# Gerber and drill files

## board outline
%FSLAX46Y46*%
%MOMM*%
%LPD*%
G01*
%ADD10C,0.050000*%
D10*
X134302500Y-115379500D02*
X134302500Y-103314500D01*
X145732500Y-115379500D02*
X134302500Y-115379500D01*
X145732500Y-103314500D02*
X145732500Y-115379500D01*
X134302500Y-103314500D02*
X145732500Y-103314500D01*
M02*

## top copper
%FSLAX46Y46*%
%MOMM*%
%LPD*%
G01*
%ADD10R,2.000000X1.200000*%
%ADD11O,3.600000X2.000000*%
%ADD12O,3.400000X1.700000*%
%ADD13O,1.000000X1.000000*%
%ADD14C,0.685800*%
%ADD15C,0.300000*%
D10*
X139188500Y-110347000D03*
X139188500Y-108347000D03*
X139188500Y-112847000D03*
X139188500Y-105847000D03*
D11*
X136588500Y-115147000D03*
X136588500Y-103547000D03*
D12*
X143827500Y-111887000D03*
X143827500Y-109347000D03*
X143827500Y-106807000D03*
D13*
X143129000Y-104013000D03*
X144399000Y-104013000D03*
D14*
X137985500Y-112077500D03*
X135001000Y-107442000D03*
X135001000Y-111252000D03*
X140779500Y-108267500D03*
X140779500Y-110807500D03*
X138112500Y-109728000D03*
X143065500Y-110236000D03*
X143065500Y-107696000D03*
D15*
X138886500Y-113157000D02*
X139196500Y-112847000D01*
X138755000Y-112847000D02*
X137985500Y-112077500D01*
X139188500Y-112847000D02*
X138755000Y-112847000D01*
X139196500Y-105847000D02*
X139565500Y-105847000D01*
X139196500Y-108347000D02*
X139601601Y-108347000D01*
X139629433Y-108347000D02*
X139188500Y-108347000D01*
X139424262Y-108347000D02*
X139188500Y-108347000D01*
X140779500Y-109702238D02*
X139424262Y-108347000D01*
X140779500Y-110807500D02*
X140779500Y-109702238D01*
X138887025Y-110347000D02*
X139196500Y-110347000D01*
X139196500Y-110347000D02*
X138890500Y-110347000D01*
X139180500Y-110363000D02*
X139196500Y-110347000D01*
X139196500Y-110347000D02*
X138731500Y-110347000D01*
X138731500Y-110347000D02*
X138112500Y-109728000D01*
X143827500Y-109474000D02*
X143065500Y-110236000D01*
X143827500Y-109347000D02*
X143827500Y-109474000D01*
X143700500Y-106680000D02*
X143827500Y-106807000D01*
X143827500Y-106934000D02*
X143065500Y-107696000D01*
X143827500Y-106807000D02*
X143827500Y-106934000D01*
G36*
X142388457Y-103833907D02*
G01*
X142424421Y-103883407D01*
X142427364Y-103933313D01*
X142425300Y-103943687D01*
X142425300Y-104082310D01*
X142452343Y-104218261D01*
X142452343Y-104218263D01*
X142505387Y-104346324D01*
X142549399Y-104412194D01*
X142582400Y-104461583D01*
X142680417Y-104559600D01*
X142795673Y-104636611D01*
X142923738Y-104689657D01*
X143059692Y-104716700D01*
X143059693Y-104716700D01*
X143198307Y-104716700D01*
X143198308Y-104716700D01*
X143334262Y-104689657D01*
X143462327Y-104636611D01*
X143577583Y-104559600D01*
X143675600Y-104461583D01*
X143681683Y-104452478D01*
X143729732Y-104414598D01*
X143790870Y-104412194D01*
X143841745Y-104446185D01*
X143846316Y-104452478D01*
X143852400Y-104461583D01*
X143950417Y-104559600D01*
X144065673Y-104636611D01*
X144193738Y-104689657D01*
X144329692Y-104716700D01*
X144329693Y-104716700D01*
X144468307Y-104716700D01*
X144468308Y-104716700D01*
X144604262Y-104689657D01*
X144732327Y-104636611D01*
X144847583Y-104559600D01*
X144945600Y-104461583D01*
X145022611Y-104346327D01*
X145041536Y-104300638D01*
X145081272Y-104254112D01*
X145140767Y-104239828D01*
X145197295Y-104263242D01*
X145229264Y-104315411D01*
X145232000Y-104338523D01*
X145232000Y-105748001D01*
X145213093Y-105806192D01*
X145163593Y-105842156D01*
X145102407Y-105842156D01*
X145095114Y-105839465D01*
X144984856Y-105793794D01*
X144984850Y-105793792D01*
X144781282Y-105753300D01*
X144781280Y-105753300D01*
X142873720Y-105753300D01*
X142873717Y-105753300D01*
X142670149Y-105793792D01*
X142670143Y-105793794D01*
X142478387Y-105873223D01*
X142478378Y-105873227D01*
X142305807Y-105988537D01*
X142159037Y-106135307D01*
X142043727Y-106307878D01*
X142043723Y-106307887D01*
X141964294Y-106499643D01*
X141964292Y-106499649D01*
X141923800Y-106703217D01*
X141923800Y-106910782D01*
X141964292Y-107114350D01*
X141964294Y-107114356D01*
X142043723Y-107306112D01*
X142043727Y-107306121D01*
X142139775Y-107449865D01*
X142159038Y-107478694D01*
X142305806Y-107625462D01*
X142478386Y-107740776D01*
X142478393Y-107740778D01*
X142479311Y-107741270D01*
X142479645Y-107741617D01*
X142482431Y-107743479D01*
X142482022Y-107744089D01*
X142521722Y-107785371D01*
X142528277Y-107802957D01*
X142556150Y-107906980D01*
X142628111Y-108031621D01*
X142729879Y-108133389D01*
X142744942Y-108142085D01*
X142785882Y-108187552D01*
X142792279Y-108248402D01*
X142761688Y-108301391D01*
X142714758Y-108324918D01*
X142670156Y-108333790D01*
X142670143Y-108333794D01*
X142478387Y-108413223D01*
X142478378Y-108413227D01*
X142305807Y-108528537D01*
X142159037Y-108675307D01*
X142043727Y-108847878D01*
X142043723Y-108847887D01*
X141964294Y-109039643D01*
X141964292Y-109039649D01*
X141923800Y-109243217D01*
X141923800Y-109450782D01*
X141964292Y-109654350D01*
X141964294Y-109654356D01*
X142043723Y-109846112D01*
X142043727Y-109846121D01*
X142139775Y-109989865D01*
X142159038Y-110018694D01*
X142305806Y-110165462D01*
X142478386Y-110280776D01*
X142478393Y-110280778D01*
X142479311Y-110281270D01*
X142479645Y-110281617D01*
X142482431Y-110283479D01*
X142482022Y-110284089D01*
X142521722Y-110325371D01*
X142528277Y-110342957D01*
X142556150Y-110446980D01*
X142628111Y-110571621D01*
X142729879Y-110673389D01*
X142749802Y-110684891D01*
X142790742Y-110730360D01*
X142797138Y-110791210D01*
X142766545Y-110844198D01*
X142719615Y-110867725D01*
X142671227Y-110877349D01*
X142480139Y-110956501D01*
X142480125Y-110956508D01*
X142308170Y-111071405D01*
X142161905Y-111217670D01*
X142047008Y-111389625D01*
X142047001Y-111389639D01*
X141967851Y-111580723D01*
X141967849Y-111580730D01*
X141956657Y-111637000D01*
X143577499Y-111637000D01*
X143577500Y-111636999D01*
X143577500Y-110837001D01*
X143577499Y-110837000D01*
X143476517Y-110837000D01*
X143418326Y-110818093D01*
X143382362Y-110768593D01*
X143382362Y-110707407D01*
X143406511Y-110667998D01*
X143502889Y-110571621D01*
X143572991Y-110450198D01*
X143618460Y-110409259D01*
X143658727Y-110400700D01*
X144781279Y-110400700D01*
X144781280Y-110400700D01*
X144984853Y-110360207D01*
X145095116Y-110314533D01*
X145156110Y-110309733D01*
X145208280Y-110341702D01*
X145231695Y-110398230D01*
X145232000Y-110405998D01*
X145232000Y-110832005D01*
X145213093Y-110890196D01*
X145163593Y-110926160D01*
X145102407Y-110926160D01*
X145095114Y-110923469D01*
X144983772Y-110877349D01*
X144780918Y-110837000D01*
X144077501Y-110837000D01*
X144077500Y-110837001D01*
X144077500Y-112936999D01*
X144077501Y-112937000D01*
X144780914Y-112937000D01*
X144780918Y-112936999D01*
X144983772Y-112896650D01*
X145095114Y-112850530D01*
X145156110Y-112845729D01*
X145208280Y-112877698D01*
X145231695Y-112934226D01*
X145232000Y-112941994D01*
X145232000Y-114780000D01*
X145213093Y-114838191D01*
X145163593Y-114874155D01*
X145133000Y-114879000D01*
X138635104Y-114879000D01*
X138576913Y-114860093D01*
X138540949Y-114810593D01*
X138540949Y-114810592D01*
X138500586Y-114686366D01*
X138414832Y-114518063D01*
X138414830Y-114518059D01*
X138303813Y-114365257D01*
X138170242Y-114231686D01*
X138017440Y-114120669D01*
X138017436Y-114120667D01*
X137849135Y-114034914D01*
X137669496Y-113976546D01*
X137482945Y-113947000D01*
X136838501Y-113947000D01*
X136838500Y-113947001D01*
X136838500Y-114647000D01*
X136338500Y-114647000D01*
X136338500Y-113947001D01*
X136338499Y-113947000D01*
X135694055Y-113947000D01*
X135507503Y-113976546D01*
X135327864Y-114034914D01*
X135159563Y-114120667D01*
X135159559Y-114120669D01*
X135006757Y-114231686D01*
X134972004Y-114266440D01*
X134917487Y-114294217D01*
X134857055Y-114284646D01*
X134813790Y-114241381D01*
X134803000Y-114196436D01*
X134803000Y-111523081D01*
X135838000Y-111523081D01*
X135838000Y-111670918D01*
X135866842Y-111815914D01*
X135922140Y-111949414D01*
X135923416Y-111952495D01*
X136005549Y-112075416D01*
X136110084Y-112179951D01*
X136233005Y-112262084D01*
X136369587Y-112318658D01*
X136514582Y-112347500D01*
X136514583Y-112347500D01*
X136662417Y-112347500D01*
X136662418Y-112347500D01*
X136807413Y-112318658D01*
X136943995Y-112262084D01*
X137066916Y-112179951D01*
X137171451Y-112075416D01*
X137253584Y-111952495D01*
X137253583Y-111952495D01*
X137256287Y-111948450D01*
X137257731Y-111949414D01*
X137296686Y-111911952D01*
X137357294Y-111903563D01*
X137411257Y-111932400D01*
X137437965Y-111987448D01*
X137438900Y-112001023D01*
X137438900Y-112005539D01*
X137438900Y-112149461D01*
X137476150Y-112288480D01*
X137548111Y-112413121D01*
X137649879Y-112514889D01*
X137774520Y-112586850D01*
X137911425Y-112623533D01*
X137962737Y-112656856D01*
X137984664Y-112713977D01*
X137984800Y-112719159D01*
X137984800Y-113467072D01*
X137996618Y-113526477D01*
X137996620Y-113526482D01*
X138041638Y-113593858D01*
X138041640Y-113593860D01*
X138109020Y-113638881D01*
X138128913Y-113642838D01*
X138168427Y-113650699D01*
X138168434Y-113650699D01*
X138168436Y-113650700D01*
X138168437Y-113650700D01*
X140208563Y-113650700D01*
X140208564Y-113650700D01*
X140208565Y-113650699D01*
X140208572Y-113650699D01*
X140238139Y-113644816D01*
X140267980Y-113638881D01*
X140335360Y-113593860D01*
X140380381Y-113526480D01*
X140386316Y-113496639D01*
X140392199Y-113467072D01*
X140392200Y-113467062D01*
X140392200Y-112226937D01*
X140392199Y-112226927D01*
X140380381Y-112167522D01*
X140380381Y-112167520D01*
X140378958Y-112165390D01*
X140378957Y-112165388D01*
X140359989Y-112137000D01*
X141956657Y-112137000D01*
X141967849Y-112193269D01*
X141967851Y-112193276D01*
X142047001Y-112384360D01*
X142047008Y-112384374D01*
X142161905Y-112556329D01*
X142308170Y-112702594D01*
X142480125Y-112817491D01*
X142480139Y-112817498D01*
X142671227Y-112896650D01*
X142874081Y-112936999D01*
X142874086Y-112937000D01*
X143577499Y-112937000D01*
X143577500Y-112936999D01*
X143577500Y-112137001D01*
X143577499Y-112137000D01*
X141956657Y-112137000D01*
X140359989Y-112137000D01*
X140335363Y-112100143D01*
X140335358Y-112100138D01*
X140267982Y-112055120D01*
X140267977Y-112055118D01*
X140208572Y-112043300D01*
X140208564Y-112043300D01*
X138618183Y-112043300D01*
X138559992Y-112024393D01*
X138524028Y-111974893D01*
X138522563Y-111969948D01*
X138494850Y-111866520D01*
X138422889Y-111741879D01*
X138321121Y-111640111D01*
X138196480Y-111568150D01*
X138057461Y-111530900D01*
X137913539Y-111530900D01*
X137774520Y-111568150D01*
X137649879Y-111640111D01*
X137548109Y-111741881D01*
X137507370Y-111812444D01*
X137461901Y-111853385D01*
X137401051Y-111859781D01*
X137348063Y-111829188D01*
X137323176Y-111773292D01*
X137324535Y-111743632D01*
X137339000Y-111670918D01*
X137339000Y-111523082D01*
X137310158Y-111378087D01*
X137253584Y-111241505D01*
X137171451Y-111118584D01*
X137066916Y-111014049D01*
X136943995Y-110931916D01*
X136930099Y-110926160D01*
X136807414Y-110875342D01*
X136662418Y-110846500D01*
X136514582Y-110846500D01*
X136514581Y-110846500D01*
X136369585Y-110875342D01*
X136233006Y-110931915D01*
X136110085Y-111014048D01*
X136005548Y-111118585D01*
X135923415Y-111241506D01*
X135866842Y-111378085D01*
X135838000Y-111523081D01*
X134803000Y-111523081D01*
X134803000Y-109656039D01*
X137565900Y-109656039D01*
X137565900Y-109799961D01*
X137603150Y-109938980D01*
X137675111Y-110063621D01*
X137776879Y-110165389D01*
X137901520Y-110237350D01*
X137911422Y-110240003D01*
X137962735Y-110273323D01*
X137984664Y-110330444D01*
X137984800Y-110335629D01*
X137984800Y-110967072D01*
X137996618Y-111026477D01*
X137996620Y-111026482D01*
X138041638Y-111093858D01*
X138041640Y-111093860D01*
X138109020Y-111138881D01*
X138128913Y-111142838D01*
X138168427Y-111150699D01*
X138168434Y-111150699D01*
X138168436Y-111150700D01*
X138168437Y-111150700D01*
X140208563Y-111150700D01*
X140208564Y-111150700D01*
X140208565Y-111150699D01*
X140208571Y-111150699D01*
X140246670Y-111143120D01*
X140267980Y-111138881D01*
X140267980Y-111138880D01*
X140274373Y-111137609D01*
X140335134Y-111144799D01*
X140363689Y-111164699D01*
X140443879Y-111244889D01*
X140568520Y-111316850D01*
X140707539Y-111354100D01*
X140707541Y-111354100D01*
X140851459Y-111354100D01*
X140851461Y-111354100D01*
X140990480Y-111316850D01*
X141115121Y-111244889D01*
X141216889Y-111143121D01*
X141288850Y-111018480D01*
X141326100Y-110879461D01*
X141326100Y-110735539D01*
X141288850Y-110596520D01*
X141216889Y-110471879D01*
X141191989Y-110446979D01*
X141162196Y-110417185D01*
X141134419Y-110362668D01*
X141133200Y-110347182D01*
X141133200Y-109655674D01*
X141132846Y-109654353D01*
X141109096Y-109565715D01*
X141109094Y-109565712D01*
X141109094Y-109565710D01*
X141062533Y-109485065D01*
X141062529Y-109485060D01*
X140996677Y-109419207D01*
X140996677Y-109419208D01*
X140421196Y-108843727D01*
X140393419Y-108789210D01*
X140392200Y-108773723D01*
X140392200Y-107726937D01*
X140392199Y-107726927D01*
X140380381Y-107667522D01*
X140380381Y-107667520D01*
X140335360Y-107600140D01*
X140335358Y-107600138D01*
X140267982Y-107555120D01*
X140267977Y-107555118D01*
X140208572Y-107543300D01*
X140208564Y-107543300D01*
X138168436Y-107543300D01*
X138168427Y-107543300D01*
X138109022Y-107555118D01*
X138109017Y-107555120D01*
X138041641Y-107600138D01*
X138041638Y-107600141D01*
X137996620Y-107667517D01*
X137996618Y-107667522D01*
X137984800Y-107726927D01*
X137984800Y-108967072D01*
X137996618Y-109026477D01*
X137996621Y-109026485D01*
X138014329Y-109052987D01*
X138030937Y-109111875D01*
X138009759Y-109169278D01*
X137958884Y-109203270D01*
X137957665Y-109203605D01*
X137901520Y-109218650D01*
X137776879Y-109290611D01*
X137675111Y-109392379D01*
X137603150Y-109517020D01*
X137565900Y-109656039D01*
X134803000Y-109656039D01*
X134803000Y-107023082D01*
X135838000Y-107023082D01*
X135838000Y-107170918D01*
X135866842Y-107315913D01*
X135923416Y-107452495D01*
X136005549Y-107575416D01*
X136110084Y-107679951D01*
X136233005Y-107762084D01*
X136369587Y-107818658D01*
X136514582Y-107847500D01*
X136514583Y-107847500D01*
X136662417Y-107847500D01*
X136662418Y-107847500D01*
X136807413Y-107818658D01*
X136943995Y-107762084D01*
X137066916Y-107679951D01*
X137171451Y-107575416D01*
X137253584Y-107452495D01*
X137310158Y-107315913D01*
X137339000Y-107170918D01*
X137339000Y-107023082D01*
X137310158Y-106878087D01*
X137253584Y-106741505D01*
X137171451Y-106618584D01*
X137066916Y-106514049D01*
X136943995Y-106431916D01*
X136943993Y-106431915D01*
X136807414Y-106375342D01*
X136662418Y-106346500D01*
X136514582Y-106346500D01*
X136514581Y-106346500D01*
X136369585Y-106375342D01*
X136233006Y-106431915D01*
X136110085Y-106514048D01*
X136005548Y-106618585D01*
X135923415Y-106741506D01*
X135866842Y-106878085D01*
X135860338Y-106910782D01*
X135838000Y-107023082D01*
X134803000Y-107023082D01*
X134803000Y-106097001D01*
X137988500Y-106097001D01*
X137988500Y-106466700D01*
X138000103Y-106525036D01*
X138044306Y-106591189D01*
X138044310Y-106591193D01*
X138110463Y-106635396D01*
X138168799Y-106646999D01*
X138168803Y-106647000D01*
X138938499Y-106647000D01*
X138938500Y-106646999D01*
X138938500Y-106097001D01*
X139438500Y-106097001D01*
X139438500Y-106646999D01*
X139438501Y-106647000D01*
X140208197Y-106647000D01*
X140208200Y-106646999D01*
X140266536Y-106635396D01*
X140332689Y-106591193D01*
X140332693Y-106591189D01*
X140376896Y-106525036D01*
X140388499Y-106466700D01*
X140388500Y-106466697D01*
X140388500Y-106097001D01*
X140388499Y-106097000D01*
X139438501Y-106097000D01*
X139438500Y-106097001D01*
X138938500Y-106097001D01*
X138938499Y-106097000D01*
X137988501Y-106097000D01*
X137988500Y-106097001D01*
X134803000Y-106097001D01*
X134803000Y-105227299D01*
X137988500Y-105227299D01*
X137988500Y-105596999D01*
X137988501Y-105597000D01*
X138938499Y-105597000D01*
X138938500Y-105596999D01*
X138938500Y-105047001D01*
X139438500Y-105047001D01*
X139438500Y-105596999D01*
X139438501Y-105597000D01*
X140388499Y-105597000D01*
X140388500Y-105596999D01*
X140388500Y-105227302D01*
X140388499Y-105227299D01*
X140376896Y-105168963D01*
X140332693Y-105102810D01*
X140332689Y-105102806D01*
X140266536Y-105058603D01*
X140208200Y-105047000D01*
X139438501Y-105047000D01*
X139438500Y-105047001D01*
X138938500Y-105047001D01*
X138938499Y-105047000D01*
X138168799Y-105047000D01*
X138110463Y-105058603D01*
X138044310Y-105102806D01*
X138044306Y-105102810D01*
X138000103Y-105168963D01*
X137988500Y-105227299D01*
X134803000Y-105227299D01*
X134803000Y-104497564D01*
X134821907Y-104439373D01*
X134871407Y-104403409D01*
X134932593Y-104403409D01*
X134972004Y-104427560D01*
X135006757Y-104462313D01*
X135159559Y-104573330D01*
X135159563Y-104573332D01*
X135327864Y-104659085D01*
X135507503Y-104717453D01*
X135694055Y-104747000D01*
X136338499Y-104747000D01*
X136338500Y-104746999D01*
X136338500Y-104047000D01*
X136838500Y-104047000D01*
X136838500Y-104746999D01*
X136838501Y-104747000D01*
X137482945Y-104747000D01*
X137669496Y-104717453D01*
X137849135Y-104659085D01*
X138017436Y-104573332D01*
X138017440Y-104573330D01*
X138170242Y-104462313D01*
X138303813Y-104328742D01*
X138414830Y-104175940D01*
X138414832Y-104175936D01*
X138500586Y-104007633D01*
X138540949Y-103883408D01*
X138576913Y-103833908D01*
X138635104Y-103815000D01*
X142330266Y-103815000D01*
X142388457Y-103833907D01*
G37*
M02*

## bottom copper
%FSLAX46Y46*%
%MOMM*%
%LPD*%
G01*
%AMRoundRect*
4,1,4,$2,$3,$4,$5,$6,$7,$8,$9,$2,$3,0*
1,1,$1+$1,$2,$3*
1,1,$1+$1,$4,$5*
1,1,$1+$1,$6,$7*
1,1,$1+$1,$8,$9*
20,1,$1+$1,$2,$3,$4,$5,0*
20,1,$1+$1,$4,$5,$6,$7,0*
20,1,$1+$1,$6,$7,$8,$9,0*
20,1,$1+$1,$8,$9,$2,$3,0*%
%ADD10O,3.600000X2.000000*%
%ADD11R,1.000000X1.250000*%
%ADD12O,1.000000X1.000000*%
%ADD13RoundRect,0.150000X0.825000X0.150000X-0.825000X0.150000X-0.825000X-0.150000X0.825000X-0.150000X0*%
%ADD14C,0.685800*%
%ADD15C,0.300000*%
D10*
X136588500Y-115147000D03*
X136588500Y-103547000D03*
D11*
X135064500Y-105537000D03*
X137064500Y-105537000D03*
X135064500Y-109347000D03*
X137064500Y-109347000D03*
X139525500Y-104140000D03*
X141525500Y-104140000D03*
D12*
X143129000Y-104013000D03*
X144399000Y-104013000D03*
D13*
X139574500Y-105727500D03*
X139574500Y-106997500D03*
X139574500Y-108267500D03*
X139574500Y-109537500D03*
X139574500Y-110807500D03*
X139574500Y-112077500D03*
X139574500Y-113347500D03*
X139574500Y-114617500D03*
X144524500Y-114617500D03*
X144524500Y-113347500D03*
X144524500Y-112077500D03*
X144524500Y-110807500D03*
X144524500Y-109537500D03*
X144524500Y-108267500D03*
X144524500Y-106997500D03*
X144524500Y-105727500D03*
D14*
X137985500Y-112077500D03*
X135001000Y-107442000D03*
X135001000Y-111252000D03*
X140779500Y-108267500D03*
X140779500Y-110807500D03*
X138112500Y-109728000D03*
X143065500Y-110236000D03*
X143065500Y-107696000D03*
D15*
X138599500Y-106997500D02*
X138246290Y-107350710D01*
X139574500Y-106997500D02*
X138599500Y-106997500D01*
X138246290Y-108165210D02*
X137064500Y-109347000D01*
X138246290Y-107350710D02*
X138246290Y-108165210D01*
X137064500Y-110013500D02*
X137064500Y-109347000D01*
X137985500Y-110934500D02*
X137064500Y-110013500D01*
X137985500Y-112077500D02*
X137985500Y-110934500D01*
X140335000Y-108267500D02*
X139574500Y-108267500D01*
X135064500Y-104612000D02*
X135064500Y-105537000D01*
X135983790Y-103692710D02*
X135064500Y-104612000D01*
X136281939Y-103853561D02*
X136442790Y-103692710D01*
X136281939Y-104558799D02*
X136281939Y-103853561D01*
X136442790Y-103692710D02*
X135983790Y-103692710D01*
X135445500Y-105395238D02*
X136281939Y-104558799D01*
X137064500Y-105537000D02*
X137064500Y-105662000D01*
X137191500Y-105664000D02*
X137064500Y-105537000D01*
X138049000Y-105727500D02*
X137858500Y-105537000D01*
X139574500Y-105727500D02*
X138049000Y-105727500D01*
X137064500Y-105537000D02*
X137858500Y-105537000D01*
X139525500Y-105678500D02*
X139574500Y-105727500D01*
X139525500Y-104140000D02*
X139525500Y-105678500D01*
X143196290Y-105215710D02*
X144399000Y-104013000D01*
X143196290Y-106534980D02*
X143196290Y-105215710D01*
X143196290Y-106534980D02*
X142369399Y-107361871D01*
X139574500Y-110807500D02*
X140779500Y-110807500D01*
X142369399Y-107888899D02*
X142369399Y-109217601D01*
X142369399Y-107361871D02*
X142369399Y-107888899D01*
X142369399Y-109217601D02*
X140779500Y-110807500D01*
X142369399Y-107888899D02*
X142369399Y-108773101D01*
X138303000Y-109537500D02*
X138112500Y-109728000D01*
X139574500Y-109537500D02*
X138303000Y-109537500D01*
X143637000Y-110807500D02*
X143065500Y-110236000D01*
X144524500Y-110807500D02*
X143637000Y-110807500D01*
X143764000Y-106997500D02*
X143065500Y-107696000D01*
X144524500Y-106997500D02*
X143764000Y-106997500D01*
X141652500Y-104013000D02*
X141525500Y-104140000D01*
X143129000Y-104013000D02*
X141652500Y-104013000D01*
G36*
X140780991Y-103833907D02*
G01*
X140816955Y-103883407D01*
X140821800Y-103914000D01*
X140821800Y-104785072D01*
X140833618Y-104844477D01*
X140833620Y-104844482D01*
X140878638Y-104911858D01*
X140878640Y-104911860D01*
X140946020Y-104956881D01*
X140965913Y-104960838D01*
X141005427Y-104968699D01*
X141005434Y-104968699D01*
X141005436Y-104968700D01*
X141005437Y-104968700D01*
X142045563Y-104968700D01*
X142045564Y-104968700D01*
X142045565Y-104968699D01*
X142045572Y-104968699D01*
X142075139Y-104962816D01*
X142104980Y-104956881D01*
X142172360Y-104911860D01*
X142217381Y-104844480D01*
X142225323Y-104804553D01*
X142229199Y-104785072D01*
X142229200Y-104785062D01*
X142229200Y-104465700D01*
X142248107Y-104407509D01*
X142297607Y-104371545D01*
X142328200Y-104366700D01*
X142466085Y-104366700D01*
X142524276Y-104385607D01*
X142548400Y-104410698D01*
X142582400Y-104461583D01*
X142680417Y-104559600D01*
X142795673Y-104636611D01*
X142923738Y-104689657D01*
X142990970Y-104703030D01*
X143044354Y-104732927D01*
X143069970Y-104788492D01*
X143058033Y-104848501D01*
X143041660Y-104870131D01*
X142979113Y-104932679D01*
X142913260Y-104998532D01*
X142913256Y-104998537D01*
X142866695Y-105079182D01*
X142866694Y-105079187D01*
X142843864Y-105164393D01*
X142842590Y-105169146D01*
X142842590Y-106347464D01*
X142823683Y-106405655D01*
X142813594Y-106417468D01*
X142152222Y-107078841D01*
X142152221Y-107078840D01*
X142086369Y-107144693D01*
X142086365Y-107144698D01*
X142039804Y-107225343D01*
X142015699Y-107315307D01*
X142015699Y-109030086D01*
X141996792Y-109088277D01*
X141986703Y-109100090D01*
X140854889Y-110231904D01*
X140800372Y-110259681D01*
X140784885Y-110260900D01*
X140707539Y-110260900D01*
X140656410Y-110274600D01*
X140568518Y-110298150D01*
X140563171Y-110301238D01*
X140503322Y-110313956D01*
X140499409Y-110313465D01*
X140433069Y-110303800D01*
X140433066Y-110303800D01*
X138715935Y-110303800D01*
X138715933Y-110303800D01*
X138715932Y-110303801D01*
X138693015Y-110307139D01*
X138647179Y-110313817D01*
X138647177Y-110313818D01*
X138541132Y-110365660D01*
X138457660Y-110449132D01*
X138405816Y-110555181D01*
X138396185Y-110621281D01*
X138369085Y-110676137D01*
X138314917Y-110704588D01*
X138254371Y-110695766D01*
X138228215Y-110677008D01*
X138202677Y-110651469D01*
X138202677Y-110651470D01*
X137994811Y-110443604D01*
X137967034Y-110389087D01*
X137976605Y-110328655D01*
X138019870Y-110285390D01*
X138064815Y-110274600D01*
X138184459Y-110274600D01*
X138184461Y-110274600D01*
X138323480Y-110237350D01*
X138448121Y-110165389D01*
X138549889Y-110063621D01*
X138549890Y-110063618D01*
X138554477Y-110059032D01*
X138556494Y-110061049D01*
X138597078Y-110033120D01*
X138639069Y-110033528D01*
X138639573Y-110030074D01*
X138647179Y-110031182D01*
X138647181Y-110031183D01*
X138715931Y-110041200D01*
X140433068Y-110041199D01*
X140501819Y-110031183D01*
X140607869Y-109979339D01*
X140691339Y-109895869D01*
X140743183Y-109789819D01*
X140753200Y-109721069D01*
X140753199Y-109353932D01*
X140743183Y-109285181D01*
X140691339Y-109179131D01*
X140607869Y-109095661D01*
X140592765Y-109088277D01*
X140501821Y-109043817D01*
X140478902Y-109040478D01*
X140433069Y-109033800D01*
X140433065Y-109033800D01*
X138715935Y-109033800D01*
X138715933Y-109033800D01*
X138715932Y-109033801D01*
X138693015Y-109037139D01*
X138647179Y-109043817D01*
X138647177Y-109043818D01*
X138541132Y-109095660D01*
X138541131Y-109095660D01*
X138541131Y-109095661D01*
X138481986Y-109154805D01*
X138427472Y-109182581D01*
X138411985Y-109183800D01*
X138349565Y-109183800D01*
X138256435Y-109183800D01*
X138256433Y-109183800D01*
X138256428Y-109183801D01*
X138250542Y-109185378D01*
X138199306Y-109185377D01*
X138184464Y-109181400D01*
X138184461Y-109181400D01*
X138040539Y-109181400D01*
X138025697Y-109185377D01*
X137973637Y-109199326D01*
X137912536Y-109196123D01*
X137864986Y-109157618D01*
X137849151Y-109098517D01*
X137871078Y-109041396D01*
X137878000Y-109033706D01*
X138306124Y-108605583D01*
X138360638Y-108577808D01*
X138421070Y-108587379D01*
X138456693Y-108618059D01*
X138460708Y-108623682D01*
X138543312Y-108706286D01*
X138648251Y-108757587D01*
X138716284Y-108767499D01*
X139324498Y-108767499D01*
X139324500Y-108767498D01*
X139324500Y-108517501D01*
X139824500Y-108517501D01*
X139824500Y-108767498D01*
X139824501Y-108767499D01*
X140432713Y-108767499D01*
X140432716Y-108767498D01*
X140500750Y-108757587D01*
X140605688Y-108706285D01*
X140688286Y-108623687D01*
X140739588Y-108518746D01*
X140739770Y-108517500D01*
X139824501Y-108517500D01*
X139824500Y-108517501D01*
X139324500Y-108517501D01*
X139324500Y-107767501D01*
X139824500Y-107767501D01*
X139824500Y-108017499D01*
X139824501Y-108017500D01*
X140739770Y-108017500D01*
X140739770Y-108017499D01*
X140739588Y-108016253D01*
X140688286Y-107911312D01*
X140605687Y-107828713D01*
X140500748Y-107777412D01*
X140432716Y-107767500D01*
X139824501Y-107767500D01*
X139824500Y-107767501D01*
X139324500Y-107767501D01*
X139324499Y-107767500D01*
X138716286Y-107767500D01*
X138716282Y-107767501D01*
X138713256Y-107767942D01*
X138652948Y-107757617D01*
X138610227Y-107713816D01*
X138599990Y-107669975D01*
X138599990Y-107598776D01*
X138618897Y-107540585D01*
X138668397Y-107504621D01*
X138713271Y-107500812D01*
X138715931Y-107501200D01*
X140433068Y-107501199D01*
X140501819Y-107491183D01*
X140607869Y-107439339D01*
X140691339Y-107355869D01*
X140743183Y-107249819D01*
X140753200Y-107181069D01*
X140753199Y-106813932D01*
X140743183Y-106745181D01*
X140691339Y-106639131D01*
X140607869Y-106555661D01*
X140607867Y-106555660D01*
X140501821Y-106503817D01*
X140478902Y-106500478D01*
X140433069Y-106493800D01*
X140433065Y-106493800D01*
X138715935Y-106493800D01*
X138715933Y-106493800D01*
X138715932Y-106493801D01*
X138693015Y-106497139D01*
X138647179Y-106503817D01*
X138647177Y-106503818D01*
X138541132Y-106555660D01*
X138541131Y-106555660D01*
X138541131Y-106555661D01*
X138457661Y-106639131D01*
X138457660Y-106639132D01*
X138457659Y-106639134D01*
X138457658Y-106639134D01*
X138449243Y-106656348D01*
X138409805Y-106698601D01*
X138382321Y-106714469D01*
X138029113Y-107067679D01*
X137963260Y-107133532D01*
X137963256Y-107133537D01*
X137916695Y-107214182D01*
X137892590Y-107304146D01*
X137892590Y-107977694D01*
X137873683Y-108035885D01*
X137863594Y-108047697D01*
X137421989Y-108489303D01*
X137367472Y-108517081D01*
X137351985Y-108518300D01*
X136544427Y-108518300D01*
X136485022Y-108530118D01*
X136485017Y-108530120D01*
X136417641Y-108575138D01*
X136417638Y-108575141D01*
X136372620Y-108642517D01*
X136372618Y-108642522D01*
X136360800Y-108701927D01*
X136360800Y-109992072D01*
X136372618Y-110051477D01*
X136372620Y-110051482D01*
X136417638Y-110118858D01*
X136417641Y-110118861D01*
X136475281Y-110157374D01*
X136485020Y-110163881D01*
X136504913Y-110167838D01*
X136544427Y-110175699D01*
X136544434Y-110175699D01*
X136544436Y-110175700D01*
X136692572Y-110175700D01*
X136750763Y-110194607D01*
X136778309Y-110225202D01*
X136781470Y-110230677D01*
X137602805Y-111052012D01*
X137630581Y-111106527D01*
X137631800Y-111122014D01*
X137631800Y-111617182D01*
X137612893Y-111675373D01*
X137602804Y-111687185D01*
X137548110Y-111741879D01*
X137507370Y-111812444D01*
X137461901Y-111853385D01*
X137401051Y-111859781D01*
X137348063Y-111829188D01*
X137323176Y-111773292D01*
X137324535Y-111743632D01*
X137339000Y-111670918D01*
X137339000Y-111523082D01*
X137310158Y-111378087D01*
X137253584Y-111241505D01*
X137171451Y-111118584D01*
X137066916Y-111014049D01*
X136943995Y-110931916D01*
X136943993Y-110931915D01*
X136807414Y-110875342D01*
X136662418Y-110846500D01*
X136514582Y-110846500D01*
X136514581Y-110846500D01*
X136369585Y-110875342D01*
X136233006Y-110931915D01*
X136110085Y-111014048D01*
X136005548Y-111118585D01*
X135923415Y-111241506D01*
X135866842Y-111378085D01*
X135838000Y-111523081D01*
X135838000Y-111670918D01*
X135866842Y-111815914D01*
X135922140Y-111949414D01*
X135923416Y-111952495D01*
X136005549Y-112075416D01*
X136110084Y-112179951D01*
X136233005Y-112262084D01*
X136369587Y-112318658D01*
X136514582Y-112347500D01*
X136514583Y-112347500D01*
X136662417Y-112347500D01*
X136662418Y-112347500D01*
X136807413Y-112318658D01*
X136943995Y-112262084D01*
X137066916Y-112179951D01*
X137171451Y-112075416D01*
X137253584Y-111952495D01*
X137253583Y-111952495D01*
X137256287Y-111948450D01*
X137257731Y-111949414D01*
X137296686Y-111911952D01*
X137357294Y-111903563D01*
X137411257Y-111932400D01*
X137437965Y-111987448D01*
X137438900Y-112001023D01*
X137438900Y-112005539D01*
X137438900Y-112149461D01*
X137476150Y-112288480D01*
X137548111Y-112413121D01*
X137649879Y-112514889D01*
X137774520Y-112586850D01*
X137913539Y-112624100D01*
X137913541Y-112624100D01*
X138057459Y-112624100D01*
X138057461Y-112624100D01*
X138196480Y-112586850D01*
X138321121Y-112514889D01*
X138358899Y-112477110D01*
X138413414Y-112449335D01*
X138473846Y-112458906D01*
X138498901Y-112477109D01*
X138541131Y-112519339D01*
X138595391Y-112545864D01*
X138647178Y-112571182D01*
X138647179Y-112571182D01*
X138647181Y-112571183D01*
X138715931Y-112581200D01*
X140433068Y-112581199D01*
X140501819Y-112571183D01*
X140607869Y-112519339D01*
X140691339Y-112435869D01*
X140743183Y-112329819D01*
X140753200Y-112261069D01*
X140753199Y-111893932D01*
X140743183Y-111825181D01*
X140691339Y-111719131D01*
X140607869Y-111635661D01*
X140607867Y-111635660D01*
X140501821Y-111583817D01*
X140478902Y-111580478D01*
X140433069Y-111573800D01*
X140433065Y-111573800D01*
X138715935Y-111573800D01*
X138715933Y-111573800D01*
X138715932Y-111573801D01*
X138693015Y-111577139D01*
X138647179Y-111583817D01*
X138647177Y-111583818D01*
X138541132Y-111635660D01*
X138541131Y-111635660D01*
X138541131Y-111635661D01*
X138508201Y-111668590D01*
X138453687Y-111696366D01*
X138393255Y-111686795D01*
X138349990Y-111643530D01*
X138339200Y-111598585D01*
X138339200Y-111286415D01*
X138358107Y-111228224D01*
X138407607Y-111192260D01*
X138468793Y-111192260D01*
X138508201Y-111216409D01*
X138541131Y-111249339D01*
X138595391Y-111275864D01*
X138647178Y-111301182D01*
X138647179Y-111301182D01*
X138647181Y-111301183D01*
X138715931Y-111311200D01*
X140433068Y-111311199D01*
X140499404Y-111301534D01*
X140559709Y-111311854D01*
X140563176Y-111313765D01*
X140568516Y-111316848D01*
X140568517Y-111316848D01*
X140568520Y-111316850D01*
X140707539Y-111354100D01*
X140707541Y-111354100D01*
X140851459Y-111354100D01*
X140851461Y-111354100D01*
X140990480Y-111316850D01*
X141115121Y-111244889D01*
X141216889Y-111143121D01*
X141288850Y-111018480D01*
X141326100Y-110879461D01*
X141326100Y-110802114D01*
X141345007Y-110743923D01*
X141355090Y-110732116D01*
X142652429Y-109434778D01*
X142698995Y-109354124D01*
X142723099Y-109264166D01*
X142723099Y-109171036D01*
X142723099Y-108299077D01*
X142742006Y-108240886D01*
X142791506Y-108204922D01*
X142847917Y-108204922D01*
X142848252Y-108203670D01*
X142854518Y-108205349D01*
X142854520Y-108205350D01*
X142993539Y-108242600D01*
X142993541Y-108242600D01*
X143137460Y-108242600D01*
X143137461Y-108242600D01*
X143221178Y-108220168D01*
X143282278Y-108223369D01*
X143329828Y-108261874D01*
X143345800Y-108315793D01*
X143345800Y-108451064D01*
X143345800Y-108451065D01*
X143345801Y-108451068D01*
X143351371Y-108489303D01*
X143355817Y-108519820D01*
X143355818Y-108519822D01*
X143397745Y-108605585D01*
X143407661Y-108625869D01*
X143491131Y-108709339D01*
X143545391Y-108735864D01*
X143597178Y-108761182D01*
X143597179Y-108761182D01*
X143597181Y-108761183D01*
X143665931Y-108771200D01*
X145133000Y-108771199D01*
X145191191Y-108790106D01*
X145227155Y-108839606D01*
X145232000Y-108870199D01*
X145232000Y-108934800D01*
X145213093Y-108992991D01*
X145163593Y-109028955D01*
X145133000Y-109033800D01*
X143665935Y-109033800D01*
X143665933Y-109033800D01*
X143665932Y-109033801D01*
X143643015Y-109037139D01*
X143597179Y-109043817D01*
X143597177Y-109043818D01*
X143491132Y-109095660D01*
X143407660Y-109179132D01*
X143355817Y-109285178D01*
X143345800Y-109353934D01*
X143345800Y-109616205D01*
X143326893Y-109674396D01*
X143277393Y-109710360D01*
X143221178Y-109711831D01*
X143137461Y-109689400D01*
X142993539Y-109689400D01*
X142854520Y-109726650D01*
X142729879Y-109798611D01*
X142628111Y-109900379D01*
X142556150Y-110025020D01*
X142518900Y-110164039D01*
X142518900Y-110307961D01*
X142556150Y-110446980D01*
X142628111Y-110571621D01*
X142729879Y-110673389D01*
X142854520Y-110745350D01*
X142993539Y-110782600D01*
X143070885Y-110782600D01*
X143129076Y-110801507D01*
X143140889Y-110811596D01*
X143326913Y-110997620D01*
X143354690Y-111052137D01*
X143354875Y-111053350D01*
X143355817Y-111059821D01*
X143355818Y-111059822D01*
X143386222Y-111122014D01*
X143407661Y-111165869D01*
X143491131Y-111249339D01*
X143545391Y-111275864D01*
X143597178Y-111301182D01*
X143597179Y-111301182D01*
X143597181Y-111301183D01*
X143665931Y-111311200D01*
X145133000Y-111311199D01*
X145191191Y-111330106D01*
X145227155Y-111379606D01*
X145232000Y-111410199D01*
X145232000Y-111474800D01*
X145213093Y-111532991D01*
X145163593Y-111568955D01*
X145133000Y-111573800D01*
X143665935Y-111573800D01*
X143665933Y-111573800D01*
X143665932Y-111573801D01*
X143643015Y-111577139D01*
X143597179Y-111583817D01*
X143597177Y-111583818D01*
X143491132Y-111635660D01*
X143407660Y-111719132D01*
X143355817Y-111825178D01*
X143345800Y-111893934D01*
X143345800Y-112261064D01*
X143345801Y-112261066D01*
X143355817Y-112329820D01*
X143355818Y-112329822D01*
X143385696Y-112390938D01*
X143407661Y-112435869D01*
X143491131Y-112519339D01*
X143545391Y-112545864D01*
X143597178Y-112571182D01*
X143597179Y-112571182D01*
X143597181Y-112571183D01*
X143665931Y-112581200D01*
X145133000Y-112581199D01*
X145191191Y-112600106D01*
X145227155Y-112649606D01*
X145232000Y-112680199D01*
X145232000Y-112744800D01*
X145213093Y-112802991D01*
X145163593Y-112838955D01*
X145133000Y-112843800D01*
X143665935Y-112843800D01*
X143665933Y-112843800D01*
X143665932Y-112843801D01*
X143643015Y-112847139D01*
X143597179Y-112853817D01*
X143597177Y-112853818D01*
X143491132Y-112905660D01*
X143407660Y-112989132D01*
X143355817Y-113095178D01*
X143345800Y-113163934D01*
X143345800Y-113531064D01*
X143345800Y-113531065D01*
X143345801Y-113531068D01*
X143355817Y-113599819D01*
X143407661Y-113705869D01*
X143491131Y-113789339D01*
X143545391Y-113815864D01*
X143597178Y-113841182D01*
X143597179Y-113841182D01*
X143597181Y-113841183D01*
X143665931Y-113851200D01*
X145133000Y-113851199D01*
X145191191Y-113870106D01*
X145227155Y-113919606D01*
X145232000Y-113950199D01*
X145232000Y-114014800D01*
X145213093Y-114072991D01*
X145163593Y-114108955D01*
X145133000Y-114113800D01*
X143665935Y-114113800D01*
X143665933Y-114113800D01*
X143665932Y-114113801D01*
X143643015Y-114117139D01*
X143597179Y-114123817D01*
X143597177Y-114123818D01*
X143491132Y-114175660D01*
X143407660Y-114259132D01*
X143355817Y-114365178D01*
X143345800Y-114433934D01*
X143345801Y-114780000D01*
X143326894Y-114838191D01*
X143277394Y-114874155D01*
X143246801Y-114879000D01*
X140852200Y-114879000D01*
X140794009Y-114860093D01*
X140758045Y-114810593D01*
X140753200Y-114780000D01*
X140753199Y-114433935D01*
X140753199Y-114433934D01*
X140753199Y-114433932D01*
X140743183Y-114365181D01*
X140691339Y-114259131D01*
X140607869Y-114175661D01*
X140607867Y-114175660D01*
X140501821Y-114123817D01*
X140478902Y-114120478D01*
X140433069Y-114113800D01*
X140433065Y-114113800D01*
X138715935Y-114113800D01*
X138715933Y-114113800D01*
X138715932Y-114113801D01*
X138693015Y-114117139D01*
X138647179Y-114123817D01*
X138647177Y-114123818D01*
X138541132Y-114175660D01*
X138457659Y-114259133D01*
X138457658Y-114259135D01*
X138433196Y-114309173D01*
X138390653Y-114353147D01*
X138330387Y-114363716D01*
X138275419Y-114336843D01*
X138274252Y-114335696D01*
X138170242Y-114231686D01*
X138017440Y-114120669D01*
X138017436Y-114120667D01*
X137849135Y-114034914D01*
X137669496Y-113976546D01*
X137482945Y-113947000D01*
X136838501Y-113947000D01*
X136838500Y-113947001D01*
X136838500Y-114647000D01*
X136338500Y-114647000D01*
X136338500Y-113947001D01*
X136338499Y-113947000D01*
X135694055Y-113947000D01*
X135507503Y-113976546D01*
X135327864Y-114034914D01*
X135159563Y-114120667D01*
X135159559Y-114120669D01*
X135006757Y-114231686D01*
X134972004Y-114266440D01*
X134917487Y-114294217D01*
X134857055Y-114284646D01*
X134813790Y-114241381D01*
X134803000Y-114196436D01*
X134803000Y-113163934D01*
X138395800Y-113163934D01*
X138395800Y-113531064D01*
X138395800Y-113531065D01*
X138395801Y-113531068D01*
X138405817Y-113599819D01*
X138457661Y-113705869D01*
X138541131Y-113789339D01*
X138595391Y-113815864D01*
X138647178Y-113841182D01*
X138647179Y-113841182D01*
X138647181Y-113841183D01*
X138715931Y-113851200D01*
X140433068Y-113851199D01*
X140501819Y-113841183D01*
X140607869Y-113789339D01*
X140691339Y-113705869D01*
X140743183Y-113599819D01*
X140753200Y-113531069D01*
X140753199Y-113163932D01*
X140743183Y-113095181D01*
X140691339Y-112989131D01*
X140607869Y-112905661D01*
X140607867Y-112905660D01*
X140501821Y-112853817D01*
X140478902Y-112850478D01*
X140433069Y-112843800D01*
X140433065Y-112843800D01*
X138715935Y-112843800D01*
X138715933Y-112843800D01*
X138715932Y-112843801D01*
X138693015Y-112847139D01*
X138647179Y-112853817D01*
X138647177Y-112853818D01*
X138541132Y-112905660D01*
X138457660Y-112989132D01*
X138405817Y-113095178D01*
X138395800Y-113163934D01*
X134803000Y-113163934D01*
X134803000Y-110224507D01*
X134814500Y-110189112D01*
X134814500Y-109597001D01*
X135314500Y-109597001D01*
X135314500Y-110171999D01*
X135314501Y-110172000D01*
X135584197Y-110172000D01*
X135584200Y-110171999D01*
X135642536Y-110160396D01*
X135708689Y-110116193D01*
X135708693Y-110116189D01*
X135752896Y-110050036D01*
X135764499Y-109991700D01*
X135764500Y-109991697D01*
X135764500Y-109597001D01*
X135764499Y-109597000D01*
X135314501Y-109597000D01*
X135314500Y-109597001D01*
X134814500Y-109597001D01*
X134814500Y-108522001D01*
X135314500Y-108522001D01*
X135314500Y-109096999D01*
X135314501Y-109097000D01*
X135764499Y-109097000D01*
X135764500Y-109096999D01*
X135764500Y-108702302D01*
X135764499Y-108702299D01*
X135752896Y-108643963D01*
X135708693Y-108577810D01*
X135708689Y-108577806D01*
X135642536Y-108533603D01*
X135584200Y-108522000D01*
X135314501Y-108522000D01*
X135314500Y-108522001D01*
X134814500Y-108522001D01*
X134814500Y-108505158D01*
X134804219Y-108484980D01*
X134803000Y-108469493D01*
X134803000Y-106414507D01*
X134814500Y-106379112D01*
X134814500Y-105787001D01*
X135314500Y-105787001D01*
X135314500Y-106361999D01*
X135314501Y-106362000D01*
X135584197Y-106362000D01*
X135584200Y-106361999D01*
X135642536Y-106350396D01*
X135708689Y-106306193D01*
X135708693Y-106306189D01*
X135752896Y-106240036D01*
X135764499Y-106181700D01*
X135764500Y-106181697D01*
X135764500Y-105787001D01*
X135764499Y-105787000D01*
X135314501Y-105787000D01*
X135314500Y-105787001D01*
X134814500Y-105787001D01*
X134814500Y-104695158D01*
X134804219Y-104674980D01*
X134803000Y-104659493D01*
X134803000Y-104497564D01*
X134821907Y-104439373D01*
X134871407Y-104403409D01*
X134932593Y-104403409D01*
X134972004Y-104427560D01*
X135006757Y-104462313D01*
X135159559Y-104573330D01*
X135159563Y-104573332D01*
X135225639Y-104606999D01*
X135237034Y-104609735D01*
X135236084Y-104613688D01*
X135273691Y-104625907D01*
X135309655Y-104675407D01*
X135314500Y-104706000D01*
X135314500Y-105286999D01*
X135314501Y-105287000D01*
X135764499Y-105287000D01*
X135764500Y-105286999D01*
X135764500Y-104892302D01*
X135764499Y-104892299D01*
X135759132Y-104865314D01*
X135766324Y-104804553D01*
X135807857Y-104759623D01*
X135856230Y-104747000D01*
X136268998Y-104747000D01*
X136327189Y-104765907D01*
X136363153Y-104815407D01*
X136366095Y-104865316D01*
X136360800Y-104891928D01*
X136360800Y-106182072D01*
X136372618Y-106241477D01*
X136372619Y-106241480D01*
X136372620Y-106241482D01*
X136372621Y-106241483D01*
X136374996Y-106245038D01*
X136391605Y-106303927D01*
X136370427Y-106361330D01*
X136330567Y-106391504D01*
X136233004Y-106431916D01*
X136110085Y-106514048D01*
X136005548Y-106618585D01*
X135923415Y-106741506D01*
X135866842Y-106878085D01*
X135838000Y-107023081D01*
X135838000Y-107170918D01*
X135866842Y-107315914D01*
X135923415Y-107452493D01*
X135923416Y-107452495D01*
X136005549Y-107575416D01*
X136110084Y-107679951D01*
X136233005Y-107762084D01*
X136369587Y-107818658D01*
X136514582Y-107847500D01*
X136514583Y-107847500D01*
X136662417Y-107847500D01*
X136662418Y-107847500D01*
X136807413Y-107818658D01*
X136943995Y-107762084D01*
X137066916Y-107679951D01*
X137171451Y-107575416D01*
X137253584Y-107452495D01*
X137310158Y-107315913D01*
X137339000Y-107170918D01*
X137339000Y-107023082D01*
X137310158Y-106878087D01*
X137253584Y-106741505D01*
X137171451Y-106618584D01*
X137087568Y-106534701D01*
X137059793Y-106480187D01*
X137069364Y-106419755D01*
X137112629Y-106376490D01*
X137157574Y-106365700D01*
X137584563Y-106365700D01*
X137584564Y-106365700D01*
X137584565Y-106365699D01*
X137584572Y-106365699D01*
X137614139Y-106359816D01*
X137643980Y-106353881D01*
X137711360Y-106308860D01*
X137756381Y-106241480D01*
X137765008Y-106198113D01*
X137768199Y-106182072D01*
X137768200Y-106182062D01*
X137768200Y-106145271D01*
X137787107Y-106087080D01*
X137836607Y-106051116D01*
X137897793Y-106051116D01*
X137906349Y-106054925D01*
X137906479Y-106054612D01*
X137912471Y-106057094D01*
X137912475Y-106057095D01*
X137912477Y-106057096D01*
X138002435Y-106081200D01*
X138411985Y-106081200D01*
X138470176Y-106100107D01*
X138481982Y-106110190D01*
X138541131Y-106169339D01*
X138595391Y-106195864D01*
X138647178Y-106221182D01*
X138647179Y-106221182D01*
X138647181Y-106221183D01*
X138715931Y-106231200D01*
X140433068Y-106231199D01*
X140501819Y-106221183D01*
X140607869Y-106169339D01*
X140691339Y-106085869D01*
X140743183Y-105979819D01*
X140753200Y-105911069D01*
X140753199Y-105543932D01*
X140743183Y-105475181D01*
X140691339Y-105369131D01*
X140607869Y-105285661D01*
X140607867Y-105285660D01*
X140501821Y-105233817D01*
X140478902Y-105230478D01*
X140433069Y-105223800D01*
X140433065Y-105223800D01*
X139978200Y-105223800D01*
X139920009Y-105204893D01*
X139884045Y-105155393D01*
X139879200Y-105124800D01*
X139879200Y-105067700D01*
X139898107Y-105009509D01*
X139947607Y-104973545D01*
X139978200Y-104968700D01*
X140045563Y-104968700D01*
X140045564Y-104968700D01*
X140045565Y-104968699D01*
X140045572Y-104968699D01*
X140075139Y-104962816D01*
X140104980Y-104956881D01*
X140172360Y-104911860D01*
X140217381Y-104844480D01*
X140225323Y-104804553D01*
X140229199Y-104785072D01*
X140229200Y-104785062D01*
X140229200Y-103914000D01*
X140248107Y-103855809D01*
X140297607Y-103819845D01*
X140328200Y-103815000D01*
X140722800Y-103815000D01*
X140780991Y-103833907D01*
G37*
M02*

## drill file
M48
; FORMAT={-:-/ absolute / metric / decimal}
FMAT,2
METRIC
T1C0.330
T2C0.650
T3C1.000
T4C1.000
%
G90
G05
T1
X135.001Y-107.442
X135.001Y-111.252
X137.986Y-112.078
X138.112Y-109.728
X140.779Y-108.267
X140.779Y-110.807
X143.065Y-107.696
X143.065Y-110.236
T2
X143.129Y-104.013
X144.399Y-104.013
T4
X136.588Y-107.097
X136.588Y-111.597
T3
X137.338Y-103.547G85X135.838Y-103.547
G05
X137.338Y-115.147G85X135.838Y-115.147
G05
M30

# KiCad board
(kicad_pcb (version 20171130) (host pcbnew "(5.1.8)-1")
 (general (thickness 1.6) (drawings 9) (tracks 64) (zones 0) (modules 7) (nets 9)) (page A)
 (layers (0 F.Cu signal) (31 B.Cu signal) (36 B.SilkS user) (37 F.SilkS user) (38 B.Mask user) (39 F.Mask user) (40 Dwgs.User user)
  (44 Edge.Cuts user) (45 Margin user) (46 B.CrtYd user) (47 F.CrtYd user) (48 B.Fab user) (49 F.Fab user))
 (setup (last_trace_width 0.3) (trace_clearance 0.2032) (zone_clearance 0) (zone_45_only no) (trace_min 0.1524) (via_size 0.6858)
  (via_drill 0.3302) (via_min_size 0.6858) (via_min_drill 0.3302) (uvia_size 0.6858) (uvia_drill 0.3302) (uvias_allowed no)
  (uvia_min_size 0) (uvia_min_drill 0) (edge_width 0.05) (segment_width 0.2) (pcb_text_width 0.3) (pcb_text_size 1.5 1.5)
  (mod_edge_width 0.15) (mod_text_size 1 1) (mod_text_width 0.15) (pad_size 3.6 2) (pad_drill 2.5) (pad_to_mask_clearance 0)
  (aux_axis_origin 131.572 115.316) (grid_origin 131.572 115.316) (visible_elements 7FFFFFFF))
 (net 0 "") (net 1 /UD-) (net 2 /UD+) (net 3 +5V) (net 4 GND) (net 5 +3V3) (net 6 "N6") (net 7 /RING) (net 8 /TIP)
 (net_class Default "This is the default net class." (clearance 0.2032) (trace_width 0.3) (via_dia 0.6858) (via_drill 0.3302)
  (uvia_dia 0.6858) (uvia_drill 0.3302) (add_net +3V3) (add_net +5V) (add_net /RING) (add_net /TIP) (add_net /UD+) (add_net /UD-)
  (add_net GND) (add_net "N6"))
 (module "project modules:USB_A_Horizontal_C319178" (layer F.Cu) (at 136.5885 109.347 180)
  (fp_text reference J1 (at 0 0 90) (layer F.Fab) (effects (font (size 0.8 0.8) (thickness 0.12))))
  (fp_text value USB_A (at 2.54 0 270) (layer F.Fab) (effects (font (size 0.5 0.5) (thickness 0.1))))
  (pad 2 smd rect (at -2.6 -1 180) (size 2 1.2) (layers F.Cu F.Paste F.Mask) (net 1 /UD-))
  (pad 3 smd rect (at -2.6 1 180) (size 2 1.2) (layers F.Cu F.Paste F.Mask) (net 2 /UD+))
  (pad 1 smd rect (at -2.6 -3.5 180) (size 2 1.2) (layers F.Cu F.Paste F.Mask) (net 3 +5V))
  (pad 4 smd rect (at -2.6 3.5 180) (size 2 1.2) (layers F.Cu F.Paste F.Mask) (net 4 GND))
  (pad 5 thru_hole oval (at 0 -5.8 180) (size 3.6 2) (drill oval 2.5 1) (layers *.Cu *.Mask) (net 4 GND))
  (pad 5 thru_hole oval (at 0 5.8 180) (size 3.6 2) (drill oval 2.5 1) (layers *.Cu *.Mask) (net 4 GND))
  (pad "" np_thru_hole circle (at 0 -2.25 180) (size 1 1) (drill 1) (layers *.Cu *.Mask))
  (pad "" np_thru_hole circle (at 0 2.25 180) (size 1 1) (drill 1) (layers *.Cu *.Mask)))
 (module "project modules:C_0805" (layer B.Cu) (at 136.0645 105.537 180)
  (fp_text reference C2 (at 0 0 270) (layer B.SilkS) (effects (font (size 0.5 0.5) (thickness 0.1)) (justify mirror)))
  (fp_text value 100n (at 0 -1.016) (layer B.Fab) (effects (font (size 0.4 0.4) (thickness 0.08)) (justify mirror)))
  (pad 2 smd rect (at 1 0 180) (size 1 1.25) (layers B.Cu B.Paste B.Mask) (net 4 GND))
  (pad 1 smd rect (at -1 0 180) (size 1 1.25) (layers B.Cu B.Paste B.Mask) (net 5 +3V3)))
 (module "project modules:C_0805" (layer B.Cu) (at 136.0645 109.347 180)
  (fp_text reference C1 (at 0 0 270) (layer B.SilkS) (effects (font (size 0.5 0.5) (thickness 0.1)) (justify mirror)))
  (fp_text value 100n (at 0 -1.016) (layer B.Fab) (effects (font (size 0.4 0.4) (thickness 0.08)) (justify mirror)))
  (pad 2 smd rect (at 1 0 180) (size 1 1.25) (layers B.Cu B.Paste B.Mask) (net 4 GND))
  (pad 1 smd rect (at -1 0 180) (size 1 1.25) (layers B.Cu B.Paste B.Mask) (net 3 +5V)))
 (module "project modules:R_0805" (layer B.Cu) (at 140.5255 104.14 180)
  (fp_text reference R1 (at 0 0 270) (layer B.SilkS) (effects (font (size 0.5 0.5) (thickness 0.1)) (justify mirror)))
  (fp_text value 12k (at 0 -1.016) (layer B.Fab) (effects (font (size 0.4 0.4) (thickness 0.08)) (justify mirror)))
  (pad 2 smd rect (at 1 0 180) (size 1 1.25) (layers B.Cu B.Paste B.Mask) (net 5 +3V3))
  (pad 1 smd rect (at -1 0 180) (size 1 1.25) (layers B.Cu B.Paste B.Mask) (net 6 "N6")))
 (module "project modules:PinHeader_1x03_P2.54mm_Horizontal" (layer F.Cu) (at 143.8275 111.887 180)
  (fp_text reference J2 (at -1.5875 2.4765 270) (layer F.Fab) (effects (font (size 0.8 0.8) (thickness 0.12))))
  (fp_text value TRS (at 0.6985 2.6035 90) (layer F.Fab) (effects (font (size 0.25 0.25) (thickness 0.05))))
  (pad 1 smd oval (at 0 0 180) (size 3.4 1.7) (layers F.Cu F.Paste F.Mask) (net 4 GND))
  (pad 2 smd oval (at 0 2.54 180) (size 3.4 1.7) (layers F.Cu F.Paste F.Mask) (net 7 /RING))
  (pad 3 smd oval (at 0 5.08 180) (size 3.4 1.7) (layers F.Cu F.Paste F.Mask) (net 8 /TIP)))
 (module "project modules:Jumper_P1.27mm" (layer B.Cu) (at 143.129 104.013 270)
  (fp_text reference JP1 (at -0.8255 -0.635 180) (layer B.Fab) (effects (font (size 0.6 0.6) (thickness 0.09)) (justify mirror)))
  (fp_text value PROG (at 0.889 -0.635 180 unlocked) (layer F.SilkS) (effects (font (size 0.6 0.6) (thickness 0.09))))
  (pad 1 thru_hole oval (at 0 0 270) (size 1 1) (drill 0.65) (layers *.Cu *.Mask) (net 6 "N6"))
  (pad 2 thru_hole oval (at 0 -1.27 270) (size 1 1) (drill 0.65) (layers *.Cu *.Mask) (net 2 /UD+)))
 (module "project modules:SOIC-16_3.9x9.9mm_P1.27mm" (layer B.Cu) (at 142.0495 110.1725 180)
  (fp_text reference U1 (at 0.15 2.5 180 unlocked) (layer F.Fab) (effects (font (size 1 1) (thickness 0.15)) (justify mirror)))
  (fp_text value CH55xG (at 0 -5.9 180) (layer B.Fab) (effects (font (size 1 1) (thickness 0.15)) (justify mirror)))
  (pad 16 smd roundrect (at 2.475 4.445 180) (size 1.95 0.6) (layers B.Cu B.Paste B.Mask) (roundrect_rratio 0.25) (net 5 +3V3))
  (pad 15 smd roundrect (at 2.475 3.175 180) (size 1.95 0.6) (layers B.Cu B.Paste B.Mask) (roundrect_rratio 0.25) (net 3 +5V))
  (pad 14 smd roundrect (at 2.475 1.905 180) (size 1.95 0.6) (layers B.Cu B.Paste B.Mask) (roundrect_rratio 0.25) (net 4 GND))
  (pad 13 smd roundrect (at 2.475 0.635 180) (size 1.95 0.6) (layers B.Cu B.Paste B.Mask) (roundrect_rratio 0.25) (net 1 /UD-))
  (pad 12 smd roundrect (at 2.475 -0.635 180) (size 1.95 0.6) (layers B.Cu B.Paste B.Mask) (roundrect_rratio 0.25) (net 2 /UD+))
  (pad 11 smd roundrect (at 2.475 -1.905 180) (size 1.95 0.6) (layers B.Cu B.Paste B.Mask) (roundrect_rratio 0.25))
  (pad 10 smd roundrect (at 2.475 -3.175 180) (size 1.95 0.6) (layers B.Cu B.Paste B.Mask) (roundrect_rratio 0.25))
  (pad 9 smd roundrect (at 2.475 -4.445 180) (size 1.95 0.6) (layers B.Cu B.Paste B.Mask) (roundrect_rratio 0.25))
  (pad 8 smd roundrect (at -2.475 -4.445 180) (size 1.95 0.6) (layers B.Cu B.Paste B.Mask) (roundrect_rratio 0.25))
  (pad 7 smd roundrect (at -2.475 -3.175 180) (size 1.95 0.6) (layers B.Cu B.Paste B.Mask) (roundrect_rratio 0.25))
  (pad 6 smd roundrect (at -2.475 -1.905 180) (size 1.95 0.6) (layers B.Cu B.Paste B.Mask) (roundrect_rratio 0.25))
  (pad 5 smd roundrect (at -2.475 -0.635 180) (size 1.95 0.6) (layers B.Cu B.Paste B.Mask) (roundrect_rratio 0.25) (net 7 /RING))
  (pad 4 smd roundrect (at -2.475 0.635 180) (size 1.95 0.6) (layers B.Cu B.Paste B.Mask) (roundrect_rratio 0.25))
  (pad 3 smd roundrect (at -2.475 1.905 180) (size 1.95 0.6) (layers B.Cu B.Paste B.Mask) (roundrect_rratio 0.25))
  (pad 2 smd roundrect (at -2.475 3.175 180) (size 1.95 0.6) (layers B.Cu B.Paste B.Mask) (roundrect_rratio 0.25) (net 8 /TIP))
  (pad 1 smd roundrect (at -2.475 4.445 180) (size 1.95 0.6) (layers B.Cu B.Paste B.Mask) (roundrect_rratio 0.25)))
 (gr_line (start 134.3025 115.3795) (end 134.3025 103.3145) (angle 90) (layer Edge.Cuts) (width 0.05))
 (gr_line (start 145.7325 115.3795) (end 134.3025 115.3795) (angle 90) (layer Edge.Cuts) (width 0.05))
 (gr_line (start 145.7325 103.3145) (end 145.7325 115.3795) (angle 90) (layer Edge.Cuts) (width 0.05))
 (gr_line (start 134.3025 103.3145) (end 145.7325 103.3145) (angle 90) (layer Edge.Cuts) (width 0.05))
 (via (at 137.9855 112.0775) (size 0.6858) (drill 0.3302) (layers F.Cu B.Cu) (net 3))
 (segment (start 138.8865 113.157) (end 139.1965 112.847) (width 0.3) (layer F.Cu) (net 3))
 (segment (start 138.5995 106.9975) (end 138.24629 107.35071) (width 0.3) (layer B.Cu) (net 3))
 (segment (start 139.5745 106.9975) (end 138.5995 106.9975) (width 0.3) (layer B.Cu) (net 3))
 (segment (start 138.24629 108.16521) (end 137.0645 109.347) (width 0.3) (layer B.Cu) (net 3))
 (segment (start 138.24629 107.35071) (end 138.24629 108.16521) (width 0.3) (layer B.Cu) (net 3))
 (segment (start 137.0645 110.0135) (end 137.0645 109.347) (width 0.3) (layer B.Cu) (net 3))
 (segment (start 137.9855 110.9345) (end 137.0645 110.0135) (width 0.3) (layer B.Cu) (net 3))
 (segment (start 137.9855 112.0775) (end 137.9855 110.9345) (width 0.3) (layer B.Cu) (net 3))
 (segment (start 138.755 112.847) (end 137.9855 112.0775) (width 0.3) (layer F.Cu) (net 3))
 (segment (start 139.1885 112.847) (end 138.755 112.847) (width 0.3) (layer F.Cu) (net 3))
 (segment (start 139.1965 105.847) (end 139.5655 105.847) (width 0.3) (layer F.Cu) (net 4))
 (via (at 135.001 107.442) (size 0.6858) (drill 0.3302) (layers F.Cu B.Cu) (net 4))
 (via (at 135.001 111.252) (size 0.6858) (drill 0.3302) (layers F.Cu B.Cu) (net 4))
 (segment (start 140.335 108.2675) (end 139.5745 108.2675) (width 0.3) (layer B.Cu) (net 4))
 (via (at 140.7795 108.2675) (size 0.6858) (drill 0.3302) (layers F.Cu B.Cu) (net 4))
 (segment (start 135.0645 104.612) (end 135.0645 105.537) (width 0.3) (layer B.Cu) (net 4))
 (segment (start 135.98379 103.69271) (end 135.0645 104.612) (width 0.3) (layer B.Cu) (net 4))
 (segment (start 136.281939 103.853561) (end 136.44279 103.69271) (width 0.3) (layer B.Cu) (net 4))
 (segment (start 136.281939 104.558799) (end 136.281939 103.853561) (width 0.3) (layer B.Cu) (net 4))
 (segment (start 136.44279 103.69271) (end 135.98379 103.69271) (width 0.3) (layer B.Cu) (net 4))
 (segment (start 135.4455 105.395238) (end 136.281939 104.558799) (width 0.3) (layer B.Cu) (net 4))
 (segment (start 137.0645 105.537) (end 137.0645 105.662) (width 0.3) (layer B.Cu) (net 5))
 (segment (start 137.1915 105.664) (end 137.0645 105.537) (width 0.3) (layer B.Cu) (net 5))
 (segment (start 138.049 105.7275) (end 137.8585 105.537) (width 0.3) (layer B.Cu) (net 5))
 (segment (start 139.5745 105.7275) (end 138.049 105.7275) (width 0.3) (layer B.Cu) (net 5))
 (segment (start 137.0645 105.537) (end 137.8585 105.537) (width 0.3) (layer B.Cu) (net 5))
 (segment (start 139.5255 105.6785) (end 139.5745 105.7275) (width 0.3) (layer B.Cu) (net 5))
 (segment (start 139.5255 104.14) (end 139.5255 105.6785) (width 0.3) (layer B.Cu) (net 5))
 (via (at 140.7795 110.8075) (size 0.6858) (drill 0.3302) (layers F.Cu B.Cu) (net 2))
 (segment (start 139.1965 108.347) (end 139.601601 108.347) (width 0.3) (layer F.Cu) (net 2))
 (segment (start 143.19629 105.21571) (end 144.399 104.013) (width 0.3) (layer B.Cu) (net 2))
 (segment (start 143.19629 106.53498) (end 143.19629 105.21571) (width 0.3) (layer B.Cu) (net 2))
 (segment (start 143.19629 106.53498) (end 142.369399 107.361871) (width 0.3) (layer B.Cu) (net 2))
 (segment (start 139.629433 108.347) (end 139.1885 108.347) (width 0.3) (layer F.Cu) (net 2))
 (segment (start 139.5745 110.8075) (end 140.7795 110.8075) (width 0.3) (layer B.Cu) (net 2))
 (segment (start 142.369399 107.888899) (end 142.369399 109.217601) (width 0.3) (layer B.Cu) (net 2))
 (segment (start 142.369399 107.361871) (end 142.369399 107.888899) (width 0.3) (layer B.Cu) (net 2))
 (segment (start 142.369399 109.217601) (end 140.7795 110.8075) (width 0.3) (layer B.Cu) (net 2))
 (segment (start 142.369399 107.888899) (end 142.369399 108.773101) (width 0.3) (layer B.Cu) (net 2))
 (segment (start 139.424262 108.347) (end 139.1885 108.347) (width 0.3) (layer F.Cu) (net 2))
 (segment (start 140.7795 109.702238) (end 139.424262 108.347) (width 0.3) (layer F.Cu) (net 2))
 (segment (start 140.7795 110.8075) (end 140.7795 109.702238) (width 0.3) (layer F.Cu) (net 2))
 (segment (start 138.887025 110.347) (end 139.1965 110.347) (width 0.3) (layer F.Cu) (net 1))
 (segment (start 139.1965 110.347) (end 138.8905 110.347) (width 0.3) (layer F.Cu) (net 1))
 (segment (start 139.1805 110.363) (end 139.1965 110.347) (width 0.3) (layer F.Cu) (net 1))
 (via (at 138.1125 109.728) (size 0.6858) (drill 0.3302) (layers F.Cu B.Cu) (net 1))
 (segment (start 139.1965 110.347) (end 138.7315 110.347) (width 0.3) (layer F.Cu) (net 1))
 (segment (start 138.7315 110.347) (end 138.1125 109.728) (width 0.3) (layer F.Cu) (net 1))
 (segment (start 138.303 109.5375) (end 138.1125 109.728) (width 0.3) (layer B.Cu) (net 1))
 (segment (start 139.5745 109.5375) (end 138.303 109.5375) (width 0.3) (layer B.Cu) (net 1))
 (via (at 143.0655 110.236) (size 0.6858) (drill 0.3302) (layers F.Cu B.Cu) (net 7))
 (segment (start 143.637 110.8075) (end 143.0655 110.236) (width 0.3) (layer B.Cu) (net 7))
 (segment (start 144.5245 110.8075) (end 143.637 110.8075) (width 0.3) (layer B.Cu) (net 7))
 (segment (start 143.8275 109.474) (end 143.0655 110.236) (width 0.3) (layer F.Cu) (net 7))
 (segment (start 143.8275 109.347) (end 143.8275 109.474) (width 0.3) (layer F.Cu) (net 7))
 (via (at 143.0655 107.696) (size 0.6858) (drill 0.3302) (layers F.Cu B.Cu) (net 8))
 (segment (start 143.7005 106.68) (end 143.8275 106.807) (width 0.3) (layer F.Cu) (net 8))
 (segment (start 143.764 106.9975) (end 143.0655 107.696) (width 0.3) (layer B.Cu) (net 8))
 (segment (start 144.5245 106.9975) (end 143.764 106.9975) (width 0.3) (layer B.Cu) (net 8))
 (segment (start 143.8275 106.934) (end 143.0655 107.696) (width 0.3) (layer F.Cu) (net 8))
 (segment (start 143.8275 106.807) (end 143.8275 106.934) (width 0.3) (layer F.Cu) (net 8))
 (segment (start 141.6525 104.013) (end 141.5255 104.14) (width 0.3) (layer B.Cu) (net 6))
 (segment (start 143.129 104.013) (end 141.6525 104.013) (width 0.3) (layer B.Cu) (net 6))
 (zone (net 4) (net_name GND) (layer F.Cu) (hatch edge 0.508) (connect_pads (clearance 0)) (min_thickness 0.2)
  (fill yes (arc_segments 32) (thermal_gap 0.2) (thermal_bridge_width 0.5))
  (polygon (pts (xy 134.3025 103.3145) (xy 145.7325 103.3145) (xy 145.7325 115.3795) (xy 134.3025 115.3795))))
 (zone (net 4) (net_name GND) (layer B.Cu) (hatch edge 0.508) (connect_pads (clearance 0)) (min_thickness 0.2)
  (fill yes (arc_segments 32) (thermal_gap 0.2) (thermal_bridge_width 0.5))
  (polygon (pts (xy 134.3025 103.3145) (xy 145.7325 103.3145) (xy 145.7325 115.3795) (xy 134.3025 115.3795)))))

